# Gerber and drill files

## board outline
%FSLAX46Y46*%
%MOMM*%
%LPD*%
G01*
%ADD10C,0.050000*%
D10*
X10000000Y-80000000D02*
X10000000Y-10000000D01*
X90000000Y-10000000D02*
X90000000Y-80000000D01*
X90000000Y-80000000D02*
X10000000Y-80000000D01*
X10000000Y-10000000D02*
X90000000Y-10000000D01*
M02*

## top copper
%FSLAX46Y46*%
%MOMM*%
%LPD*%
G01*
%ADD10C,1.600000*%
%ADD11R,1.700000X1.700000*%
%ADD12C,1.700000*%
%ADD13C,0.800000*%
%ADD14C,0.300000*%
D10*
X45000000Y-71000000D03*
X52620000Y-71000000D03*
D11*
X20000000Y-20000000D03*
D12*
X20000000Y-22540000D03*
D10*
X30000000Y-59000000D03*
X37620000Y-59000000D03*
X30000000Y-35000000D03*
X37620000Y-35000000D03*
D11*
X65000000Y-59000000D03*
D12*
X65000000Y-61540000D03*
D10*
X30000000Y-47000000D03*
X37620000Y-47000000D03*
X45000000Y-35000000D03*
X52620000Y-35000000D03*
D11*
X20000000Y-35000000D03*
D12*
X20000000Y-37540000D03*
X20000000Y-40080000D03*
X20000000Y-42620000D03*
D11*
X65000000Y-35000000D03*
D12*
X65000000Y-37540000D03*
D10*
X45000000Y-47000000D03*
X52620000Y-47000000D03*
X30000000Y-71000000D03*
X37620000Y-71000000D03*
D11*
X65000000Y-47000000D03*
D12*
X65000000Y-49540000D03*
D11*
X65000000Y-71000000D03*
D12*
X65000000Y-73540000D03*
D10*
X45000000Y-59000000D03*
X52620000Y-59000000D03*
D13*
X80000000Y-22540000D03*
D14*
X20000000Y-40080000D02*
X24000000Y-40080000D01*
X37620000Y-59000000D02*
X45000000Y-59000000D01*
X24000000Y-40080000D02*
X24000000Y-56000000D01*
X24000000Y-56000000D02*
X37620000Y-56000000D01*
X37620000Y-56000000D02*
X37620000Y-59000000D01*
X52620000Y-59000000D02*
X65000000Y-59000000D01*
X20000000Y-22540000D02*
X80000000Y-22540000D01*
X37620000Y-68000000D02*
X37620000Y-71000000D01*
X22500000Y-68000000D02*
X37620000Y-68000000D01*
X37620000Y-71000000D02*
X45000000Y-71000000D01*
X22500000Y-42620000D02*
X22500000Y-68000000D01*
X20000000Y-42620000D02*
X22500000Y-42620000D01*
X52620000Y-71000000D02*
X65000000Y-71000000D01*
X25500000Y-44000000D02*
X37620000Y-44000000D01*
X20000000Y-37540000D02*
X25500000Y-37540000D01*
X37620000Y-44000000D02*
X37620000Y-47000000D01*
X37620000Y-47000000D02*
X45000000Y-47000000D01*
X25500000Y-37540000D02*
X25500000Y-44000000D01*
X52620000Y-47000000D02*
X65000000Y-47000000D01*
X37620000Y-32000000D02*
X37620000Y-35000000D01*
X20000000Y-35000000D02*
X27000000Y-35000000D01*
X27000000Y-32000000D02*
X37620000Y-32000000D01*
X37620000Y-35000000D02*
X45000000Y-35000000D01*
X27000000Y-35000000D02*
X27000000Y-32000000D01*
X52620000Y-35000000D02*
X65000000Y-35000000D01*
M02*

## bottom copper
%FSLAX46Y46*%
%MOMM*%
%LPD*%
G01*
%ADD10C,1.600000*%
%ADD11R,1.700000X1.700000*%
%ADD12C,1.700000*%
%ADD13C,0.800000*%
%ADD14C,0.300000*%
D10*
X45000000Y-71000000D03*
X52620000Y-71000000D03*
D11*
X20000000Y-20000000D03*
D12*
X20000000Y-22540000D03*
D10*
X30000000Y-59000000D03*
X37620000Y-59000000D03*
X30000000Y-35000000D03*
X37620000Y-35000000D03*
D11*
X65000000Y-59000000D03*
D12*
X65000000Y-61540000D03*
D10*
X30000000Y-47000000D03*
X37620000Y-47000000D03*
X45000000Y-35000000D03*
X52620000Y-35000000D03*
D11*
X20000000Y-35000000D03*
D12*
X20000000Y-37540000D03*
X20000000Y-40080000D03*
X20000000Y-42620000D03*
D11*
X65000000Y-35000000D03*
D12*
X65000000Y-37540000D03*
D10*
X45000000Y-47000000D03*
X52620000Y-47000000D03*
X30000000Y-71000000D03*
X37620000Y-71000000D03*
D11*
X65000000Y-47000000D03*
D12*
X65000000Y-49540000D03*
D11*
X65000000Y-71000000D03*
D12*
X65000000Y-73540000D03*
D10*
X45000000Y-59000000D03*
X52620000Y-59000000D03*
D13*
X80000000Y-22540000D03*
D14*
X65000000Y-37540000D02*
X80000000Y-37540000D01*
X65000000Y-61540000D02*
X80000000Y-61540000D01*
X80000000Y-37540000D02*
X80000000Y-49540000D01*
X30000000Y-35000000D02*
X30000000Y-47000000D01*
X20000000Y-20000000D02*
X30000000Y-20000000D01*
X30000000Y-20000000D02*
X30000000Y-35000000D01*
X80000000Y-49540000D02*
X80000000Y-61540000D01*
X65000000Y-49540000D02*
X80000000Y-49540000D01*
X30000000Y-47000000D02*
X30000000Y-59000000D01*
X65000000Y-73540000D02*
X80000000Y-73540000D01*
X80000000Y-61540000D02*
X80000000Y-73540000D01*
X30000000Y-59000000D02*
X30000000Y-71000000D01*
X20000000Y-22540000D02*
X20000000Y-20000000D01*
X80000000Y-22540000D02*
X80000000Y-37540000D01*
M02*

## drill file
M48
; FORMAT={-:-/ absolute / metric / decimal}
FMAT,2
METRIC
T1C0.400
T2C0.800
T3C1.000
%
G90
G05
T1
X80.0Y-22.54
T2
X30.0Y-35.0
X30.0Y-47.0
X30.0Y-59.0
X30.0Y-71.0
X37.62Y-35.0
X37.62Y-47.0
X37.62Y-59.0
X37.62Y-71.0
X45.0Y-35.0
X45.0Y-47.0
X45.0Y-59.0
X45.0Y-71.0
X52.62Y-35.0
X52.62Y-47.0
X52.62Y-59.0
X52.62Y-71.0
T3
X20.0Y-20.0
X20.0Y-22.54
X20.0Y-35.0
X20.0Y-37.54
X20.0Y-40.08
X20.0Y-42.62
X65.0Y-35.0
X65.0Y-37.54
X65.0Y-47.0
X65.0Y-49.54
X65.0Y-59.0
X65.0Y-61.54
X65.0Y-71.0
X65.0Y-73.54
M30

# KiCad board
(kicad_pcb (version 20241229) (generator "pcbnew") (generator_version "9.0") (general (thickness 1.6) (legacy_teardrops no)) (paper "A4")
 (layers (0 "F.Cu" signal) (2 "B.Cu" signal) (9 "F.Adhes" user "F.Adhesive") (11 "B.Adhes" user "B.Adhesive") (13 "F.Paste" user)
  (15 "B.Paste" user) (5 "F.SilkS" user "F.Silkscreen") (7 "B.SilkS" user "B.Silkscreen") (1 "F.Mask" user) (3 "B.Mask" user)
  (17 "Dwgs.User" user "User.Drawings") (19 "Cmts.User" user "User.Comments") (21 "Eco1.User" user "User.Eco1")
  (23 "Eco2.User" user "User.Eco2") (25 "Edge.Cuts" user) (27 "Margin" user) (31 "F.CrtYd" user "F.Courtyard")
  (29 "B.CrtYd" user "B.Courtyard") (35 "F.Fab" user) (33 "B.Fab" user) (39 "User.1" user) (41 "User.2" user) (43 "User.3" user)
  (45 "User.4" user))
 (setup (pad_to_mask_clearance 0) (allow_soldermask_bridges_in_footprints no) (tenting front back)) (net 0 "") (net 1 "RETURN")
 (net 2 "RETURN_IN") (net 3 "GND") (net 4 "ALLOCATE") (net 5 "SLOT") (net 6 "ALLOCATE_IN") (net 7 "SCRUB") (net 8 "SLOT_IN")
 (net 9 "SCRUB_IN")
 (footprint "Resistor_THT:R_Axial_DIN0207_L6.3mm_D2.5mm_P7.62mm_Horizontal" (layer "F.Cu") (at 45 71)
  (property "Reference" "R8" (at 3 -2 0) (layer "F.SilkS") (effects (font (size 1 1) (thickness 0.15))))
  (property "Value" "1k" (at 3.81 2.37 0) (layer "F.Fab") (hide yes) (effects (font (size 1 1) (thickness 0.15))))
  (pad "1" thru_hole circle (at 0 0) (size 1.6 1.6) (drill 0.8) (layers "*.Cu" "*.Mask") (remove_unused_layers no) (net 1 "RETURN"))
  (pad "2" thru_hole circle (at 7.62 0) (size 1.6 1.6) (drill 0.8) (layers "*.Cu" "*.Mask") (remove_unused_layers no) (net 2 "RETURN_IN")))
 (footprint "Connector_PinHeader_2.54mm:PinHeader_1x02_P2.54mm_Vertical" (layer "F.Cu") (at 20 20)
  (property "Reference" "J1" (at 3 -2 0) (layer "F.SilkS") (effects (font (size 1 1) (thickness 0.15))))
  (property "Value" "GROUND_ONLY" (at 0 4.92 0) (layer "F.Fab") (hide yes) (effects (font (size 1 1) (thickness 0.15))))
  (pad "1" thru_hole rect (at 0 0) (size 1.7 1.7) (drill 1) (layers "*.Cu" "*.Mask") (remove_unused_layers no) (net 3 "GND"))
  (pad "2" thru_hole circle (at 0 2.54) (size 1.7 1.7) (drill 1) (layers "*.Cu" "*.Mask") (remove_unused_layers no) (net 3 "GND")))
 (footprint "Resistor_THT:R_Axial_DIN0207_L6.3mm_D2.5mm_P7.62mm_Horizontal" (layer "F.Cu") (at 30 59)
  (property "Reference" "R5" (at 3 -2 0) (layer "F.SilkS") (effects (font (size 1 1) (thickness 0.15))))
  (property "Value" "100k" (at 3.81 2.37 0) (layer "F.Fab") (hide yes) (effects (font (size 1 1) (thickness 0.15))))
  (pad "1" thru_hole circle (at 0 0) (size 1.6 1.6) (drill 0.8) (layers "*.Cu" "*.Mask") (remove_unused_layers no) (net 3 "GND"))
  (pad "2" thru_hole circle (at 7.62 0) (size 1.6 1.6) (drill 0.8) (layers "*.Cu" "*.Mask") (remove_unused_layers no) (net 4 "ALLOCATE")))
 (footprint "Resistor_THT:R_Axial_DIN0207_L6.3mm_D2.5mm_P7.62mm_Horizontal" (layer "F.Cu") (at 30 35)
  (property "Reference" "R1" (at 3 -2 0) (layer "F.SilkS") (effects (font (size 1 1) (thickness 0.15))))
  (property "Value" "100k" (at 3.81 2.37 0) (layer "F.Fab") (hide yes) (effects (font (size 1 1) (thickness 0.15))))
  (pad "1" thru_hole circle (at 0 0) (size 1.6 1.6) (drill 0.8) (layers "*.Cu" "*.Mask") (remove_unused_layers no) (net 3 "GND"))
  (pad "2" thru_hole circle (at 7.62 0) (size 1.6 1.6) (drill 0.8) (layers "*.Cu" "*.Mask") (remove_unused_layers no) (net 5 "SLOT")))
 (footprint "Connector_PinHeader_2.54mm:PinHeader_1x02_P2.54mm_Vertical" (layer "F.Cu") (at 65 59)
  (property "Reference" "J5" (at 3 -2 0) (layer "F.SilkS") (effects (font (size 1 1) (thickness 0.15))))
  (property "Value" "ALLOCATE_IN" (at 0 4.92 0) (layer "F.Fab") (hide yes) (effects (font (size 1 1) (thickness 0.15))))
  (pad "1" thru_hole rect (at 0 0) (size 1.7 1.7) (drill 1) (layers "*.Cu" "*.Mask") (remove_unused_layers no) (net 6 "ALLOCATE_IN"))
  (pad "2" thru_hole circle (at 0 2.54) (size 1.7 1.7) (drill 1) (layers "*.Cu" "*.Mask") (remove_unused_layers no) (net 3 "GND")))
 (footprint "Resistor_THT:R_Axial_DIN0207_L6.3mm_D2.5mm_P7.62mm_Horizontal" (layer "F.Cu") (at 30 47)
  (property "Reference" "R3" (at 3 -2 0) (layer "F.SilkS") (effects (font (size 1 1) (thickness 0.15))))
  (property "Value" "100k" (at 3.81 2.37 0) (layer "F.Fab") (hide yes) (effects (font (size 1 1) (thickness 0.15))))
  (pad "1" thru_hole circle (at 0 0) (size 1.6 1.6) (drill 0.8) (layers "*.Cu" "*.Mask") (remove_unused_layers no) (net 3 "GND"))
  (pad "2" thru_hole circle (at 7.62 0) (size 1.6 1.6) (drill 0.8) (layers "*.Cu" "*.Mask") (remove_unused_layers no) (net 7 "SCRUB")))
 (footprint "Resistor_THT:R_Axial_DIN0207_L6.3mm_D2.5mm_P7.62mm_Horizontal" (layer "F.Cu") (at 45 35)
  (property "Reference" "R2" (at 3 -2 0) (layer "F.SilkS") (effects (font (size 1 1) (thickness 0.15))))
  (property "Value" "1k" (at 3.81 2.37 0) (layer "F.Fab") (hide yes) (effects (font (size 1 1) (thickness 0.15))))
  (pad "1" thru_hole circle (at 0 0) (size 1.6 1.6) (drill 0.8) (layers "*.Cu" "*.Mask") (remove_unused_layers no) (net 5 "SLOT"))
  (pad "2" thru_hole circle (at 7.62 0) (size 1.6 1.6) (drill 0.8) (layers "*.Cu" "*.Mask") (remove_unused_layers no) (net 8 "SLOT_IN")))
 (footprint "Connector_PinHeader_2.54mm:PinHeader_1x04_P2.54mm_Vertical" (layer "F.Cu") (at 20 35)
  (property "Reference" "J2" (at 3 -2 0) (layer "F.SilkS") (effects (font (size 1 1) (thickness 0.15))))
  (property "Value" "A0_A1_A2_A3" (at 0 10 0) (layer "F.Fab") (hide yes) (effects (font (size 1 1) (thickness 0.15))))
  (pad "1" thru_hole rect (at 0 0) (size 1.7 1.7) (drill 1) (layers "*.Cu" "*.Mask") (remove_unused_layers no) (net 5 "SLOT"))
  (pad "2" thru_hole circle (at 0 2.54) (size 1.7 1.7) (drill 1) (layers "*.Cu" "*.Mask") (remove_unused_layers no) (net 7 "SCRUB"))
  (pad "3" thru_hole circle (at 0 5.08) (size 1.7 1.7) (drill 1) (layers "*.Cu" "*.Mask") (remove_unused_layers no) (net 4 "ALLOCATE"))
  (pad "4" thru_hole circle (at 0 7.62) (size 1.7 1.7) (drill 1) (layers "*.Cu" "*.Mask") (remove_unused_layers no) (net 1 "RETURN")))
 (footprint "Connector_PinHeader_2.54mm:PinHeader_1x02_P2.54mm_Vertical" (layer "F.Cu") (at 65 35)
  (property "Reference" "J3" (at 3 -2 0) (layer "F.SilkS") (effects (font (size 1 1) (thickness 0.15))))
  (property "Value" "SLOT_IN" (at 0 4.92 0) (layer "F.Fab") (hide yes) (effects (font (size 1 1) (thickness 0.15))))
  (pad "1" thru_hole rect (at 0 0) (size 1.7 1.7) (drill 1) (layers "*.Cu" "*.Mask") (remove_unused_layers no) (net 8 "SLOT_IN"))
  (pad "2" thru_hole circle (at 0 2.54) (size 1.7 1.7) (drill 1) (layers "*.Cu" "*.Mask") (remove_unused_layers no) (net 3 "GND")))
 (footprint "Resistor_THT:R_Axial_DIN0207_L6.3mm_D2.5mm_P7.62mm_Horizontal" (layer "F.Cu") (at 45 47)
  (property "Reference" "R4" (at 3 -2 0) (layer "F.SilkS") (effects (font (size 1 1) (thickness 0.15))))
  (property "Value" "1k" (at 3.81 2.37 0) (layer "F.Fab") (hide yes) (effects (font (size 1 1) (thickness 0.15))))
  (pad "1" thru_hole circle (at 0 0) (size 1.6 1.6) (drill 0.8) (layers "*.Cu" "*.Mask") (remove_unused_layers no) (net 7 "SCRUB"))
  (pad "2" thru_hole circle (at 7.62 0) (size 1.6 1.6) (drill 0.8) (layers "*.Cu" "*.Mask") (remove_unused_layers no) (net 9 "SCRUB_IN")))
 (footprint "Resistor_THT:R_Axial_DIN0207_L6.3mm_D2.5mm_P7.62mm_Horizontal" (layer "F.Cu") (at 30 71)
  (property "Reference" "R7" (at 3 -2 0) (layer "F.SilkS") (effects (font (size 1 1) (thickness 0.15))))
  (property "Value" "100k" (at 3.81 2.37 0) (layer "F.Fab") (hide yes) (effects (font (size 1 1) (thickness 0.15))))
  (pad "1" thru_hole circle (at 0 0) (size 1.6 1.6) (drill 0.8) (layers "*.Cu" "*.Mask") (remove_unused_layers no) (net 3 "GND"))
  (pad "2" thru_hole circle (at 7.62 0) (size 1.6 1.6) (drill 0.8) (layers "*.Cu" "*.Mask") (remove_unused_layers no) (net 1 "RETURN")))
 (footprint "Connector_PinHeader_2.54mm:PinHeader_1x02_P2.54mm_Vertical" (layer "F.Cu") (at 65 47)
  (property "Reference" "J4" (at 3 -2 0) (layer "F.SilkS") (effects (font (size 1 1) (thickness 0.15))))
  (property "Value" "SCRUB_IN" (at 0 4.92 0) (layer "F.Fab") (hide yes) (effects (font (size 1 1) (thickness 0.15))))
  (pad "1" thru_hole rect (at 0 0) (size 1.7 1.7) (drill 1) (layers "*.Cu" "*.Mask") (remove_unused_layers no) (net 9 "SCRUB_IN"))
  (pad "2" thru_hole circle (at 0 2.54) (size 1.7 1.7) (drill 1) (layers "*.Cu" "*.Mask") (remove_unused_layers no) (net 3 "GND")))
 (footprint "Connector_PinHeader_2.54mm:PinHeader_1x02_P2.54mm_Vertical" (layer "F.Cu") (at 65 71)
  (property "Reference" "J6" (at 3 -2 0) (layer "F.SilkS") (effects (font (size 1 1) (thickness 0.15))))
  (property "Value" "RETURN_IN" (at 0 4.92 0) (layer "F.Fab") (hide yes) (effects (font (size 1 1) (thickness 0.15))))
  (pad "1" thru_hole rect (at 0 0) (size 1.7 1.7) (drill 1) (layers "*.Cu" "*.Mask") (remove_unused_layers no) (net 2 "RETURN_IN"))
  (pad "2" thru_hole circle (at 0 2.54) (size 1.7 1.7) (drill 1) (layers "*.Cu" "*.Mask") (remove_unused_layers no) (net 3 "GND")))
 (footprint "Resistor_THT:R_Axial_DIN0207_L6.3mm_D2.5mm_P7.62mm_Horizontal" (layer "F.Cu") (at 45 59)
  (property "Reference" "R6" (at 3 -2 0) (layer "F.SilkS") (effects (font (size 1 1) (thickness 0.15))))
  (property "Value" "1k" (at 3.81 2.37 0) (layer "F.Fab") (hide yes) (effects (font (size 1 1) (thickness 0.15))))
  (pad "1" thru_hole circle (at 0 0) (size 1.6 1.6) (drill 0.8) (layers "*.Cu" "*.Mask") (remove_unused_layers no) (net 4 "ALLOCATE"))
  (pad "2" thru_hole circle (at 7.62 0) (size 1.6 1.6) (drill 0.8) (layers "*.Cu" "*.Mask") (remove_unused_layers no) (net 6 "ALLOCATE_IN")))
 (gr_line (start 10 80) (end 10 10) (stroke (width 0.05) (type default)) (layer "Edge.Cuts"))
 (gr_line (start 90 10) (end 90 80) (stroke (width 0.05) (type default)) (layer "Edge.Cuts"))
 (gr_line (start 90 80) (end 10 80) (stroke (width 0.05) (type default)) (layer "Edge.Cuts"))
 (gr_line (start 10 10) (end 90 10) (stroke (width 0.05) (type default)) (layer "Edge.Cuts"))
 (segment (start 20 40.08) (end 24 40.08) (width 0.3) (layer "F.Cu") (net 4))
 (segment (start 37.62 59) (end 45 59) (width 0.3) (layer "F.Cu") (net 4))
 (segment (start 24 40.08) (end 24 56) (width 0.3) (layer "F.Cu") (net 4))
 (segment (start 24 56) (end 37.62 56) (width 0.3) (layer "F.Cu") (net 4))
 (segment (start 37.62 56) (end 37.62 59) (width 0.3) (layer "F.Cu") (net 4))
 (segment (start 52.62 59) (end 65 59) (width 0.3) (layer "F.Cu") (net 6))
 (segment (start 20 22.54) (end 80 22.54) (width 0.3) (layer "F.Cu") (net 3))
 (via (at 80 22.54) (size 0.8) (drill 0.4) (layers "F.Cu" "B.Cu") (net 3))
 (segment (start 65 37.54) (end 80 37.54) (width 0.3) (layer "B.Cu") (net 3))
 (segment (start 65 61.54) (end 80 61.54) (width 0.3) (layer "B.Cu") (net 3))
 (segment (start 80 37.54) (end 80 49.54) (width 0.3) (layer "B.Cu") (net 3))
 (segment (start 30 35) (end 30 47) (width 0.3) (layer "B.Cu") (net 3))
 (segment (start 20 20) (end 30 20) (width 0.3) (layer "B.Cu") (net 3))
 (segment (start 30 20) (end 30 35) (width 0.3) (layer "B.Cu") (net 3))
 (segment (start 80 49.54) (end 80 61.54) (width 0.3) (layer "B.Cu") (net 3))
 (segment (start 65 49.54) (end 80 49.54) (width 0.3) (layer "B.Cu") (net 3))
 (segment (start 30 47) (end 30 59) (width 0.3) (layer "B.Cu") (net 3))
 (segment (start 65 73.54) (end 80 73.54) (width 0.3) (layer "B.Cu") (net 3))
 (segment (start 80 61.54) (end 80 73.54) (width 0.3) (layer "B.Cu") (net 3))
 (segment (start 30 59) (end 30 71) (width 0.3) (layer "B.Cu") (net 3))
 (segment (start 20 22.54) (end 20 20) (width 0.3) (layer "B.Cu") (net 3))
 (segment (start 80 22.54) (end 80 37.54) (width 0.3) (layer "B.Cu") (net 3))
 (segment (start 37.62 68) (end 37.62 71) (width 0.3) (layer "F.Cu") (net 1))
 (segment (start 22.5 68) (end 37.62 68) (width 0.3) (layer "F.Cu") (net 1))
 (segment (start 37.62 71) (end 45 71) (width 0.3) (layer "F.Cu") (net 1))
 (segment (start 22.5 42.62) (end 22.5 68) (width 0.3) (layer "F.Cu") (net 1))
 (segment (start 20 42.62) (end 22.5 42.62) (width 0.3) (layer "F.Cu") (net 1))
 (segment (start 52.62 71) (end 65 71) (width 0.3) (layer "F.Cu") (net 2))
 (segment (start 25.5 44) (end 37.62 44) (width 0.3) (layer "F.Cu") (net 7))
 (segment (start 20 37.54) (end 25.5 37.54) (width 0.3) (layer "F.Cu") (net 7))
 (segment (start 37.62 44) (end 37.62 47) (width 0.3) (layer "F.Cu") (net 7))
 (segment (start 37.62 47) (end 45 47) (width 0.3) (layer "F.Cu") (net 7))
 (segment (start 25.5 37.54) (end 25.5 44) (width 0.3) (layer "F.Cu") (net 7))
 (segment (start 52.62 47) (end 65 47) (width 0.3) (layer "F.Cu") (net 9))
 (segment (start 37.62 32) (end 37.62 35) (width 0.3) (layer "F.Cu") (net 5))
 (segment (start 20 35) (end 27 35) (width 0.3) (layer "F.Cu") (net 5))
 (segment (start 27 32) (end 37.62 32) (width 0.3) (layer "F.Cu") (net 5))
 (segment (start 37.62 35) (end 45 35) (width 0.3) (layer "F.Cu") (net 5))
 (segment (start 27 35) (end 27 32) (width 0.3) (layer "F.Cu") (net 5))
 (segment (start 52.62 35) (end 65 35) (width 0.3) (layer "F.Cu") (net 8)))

